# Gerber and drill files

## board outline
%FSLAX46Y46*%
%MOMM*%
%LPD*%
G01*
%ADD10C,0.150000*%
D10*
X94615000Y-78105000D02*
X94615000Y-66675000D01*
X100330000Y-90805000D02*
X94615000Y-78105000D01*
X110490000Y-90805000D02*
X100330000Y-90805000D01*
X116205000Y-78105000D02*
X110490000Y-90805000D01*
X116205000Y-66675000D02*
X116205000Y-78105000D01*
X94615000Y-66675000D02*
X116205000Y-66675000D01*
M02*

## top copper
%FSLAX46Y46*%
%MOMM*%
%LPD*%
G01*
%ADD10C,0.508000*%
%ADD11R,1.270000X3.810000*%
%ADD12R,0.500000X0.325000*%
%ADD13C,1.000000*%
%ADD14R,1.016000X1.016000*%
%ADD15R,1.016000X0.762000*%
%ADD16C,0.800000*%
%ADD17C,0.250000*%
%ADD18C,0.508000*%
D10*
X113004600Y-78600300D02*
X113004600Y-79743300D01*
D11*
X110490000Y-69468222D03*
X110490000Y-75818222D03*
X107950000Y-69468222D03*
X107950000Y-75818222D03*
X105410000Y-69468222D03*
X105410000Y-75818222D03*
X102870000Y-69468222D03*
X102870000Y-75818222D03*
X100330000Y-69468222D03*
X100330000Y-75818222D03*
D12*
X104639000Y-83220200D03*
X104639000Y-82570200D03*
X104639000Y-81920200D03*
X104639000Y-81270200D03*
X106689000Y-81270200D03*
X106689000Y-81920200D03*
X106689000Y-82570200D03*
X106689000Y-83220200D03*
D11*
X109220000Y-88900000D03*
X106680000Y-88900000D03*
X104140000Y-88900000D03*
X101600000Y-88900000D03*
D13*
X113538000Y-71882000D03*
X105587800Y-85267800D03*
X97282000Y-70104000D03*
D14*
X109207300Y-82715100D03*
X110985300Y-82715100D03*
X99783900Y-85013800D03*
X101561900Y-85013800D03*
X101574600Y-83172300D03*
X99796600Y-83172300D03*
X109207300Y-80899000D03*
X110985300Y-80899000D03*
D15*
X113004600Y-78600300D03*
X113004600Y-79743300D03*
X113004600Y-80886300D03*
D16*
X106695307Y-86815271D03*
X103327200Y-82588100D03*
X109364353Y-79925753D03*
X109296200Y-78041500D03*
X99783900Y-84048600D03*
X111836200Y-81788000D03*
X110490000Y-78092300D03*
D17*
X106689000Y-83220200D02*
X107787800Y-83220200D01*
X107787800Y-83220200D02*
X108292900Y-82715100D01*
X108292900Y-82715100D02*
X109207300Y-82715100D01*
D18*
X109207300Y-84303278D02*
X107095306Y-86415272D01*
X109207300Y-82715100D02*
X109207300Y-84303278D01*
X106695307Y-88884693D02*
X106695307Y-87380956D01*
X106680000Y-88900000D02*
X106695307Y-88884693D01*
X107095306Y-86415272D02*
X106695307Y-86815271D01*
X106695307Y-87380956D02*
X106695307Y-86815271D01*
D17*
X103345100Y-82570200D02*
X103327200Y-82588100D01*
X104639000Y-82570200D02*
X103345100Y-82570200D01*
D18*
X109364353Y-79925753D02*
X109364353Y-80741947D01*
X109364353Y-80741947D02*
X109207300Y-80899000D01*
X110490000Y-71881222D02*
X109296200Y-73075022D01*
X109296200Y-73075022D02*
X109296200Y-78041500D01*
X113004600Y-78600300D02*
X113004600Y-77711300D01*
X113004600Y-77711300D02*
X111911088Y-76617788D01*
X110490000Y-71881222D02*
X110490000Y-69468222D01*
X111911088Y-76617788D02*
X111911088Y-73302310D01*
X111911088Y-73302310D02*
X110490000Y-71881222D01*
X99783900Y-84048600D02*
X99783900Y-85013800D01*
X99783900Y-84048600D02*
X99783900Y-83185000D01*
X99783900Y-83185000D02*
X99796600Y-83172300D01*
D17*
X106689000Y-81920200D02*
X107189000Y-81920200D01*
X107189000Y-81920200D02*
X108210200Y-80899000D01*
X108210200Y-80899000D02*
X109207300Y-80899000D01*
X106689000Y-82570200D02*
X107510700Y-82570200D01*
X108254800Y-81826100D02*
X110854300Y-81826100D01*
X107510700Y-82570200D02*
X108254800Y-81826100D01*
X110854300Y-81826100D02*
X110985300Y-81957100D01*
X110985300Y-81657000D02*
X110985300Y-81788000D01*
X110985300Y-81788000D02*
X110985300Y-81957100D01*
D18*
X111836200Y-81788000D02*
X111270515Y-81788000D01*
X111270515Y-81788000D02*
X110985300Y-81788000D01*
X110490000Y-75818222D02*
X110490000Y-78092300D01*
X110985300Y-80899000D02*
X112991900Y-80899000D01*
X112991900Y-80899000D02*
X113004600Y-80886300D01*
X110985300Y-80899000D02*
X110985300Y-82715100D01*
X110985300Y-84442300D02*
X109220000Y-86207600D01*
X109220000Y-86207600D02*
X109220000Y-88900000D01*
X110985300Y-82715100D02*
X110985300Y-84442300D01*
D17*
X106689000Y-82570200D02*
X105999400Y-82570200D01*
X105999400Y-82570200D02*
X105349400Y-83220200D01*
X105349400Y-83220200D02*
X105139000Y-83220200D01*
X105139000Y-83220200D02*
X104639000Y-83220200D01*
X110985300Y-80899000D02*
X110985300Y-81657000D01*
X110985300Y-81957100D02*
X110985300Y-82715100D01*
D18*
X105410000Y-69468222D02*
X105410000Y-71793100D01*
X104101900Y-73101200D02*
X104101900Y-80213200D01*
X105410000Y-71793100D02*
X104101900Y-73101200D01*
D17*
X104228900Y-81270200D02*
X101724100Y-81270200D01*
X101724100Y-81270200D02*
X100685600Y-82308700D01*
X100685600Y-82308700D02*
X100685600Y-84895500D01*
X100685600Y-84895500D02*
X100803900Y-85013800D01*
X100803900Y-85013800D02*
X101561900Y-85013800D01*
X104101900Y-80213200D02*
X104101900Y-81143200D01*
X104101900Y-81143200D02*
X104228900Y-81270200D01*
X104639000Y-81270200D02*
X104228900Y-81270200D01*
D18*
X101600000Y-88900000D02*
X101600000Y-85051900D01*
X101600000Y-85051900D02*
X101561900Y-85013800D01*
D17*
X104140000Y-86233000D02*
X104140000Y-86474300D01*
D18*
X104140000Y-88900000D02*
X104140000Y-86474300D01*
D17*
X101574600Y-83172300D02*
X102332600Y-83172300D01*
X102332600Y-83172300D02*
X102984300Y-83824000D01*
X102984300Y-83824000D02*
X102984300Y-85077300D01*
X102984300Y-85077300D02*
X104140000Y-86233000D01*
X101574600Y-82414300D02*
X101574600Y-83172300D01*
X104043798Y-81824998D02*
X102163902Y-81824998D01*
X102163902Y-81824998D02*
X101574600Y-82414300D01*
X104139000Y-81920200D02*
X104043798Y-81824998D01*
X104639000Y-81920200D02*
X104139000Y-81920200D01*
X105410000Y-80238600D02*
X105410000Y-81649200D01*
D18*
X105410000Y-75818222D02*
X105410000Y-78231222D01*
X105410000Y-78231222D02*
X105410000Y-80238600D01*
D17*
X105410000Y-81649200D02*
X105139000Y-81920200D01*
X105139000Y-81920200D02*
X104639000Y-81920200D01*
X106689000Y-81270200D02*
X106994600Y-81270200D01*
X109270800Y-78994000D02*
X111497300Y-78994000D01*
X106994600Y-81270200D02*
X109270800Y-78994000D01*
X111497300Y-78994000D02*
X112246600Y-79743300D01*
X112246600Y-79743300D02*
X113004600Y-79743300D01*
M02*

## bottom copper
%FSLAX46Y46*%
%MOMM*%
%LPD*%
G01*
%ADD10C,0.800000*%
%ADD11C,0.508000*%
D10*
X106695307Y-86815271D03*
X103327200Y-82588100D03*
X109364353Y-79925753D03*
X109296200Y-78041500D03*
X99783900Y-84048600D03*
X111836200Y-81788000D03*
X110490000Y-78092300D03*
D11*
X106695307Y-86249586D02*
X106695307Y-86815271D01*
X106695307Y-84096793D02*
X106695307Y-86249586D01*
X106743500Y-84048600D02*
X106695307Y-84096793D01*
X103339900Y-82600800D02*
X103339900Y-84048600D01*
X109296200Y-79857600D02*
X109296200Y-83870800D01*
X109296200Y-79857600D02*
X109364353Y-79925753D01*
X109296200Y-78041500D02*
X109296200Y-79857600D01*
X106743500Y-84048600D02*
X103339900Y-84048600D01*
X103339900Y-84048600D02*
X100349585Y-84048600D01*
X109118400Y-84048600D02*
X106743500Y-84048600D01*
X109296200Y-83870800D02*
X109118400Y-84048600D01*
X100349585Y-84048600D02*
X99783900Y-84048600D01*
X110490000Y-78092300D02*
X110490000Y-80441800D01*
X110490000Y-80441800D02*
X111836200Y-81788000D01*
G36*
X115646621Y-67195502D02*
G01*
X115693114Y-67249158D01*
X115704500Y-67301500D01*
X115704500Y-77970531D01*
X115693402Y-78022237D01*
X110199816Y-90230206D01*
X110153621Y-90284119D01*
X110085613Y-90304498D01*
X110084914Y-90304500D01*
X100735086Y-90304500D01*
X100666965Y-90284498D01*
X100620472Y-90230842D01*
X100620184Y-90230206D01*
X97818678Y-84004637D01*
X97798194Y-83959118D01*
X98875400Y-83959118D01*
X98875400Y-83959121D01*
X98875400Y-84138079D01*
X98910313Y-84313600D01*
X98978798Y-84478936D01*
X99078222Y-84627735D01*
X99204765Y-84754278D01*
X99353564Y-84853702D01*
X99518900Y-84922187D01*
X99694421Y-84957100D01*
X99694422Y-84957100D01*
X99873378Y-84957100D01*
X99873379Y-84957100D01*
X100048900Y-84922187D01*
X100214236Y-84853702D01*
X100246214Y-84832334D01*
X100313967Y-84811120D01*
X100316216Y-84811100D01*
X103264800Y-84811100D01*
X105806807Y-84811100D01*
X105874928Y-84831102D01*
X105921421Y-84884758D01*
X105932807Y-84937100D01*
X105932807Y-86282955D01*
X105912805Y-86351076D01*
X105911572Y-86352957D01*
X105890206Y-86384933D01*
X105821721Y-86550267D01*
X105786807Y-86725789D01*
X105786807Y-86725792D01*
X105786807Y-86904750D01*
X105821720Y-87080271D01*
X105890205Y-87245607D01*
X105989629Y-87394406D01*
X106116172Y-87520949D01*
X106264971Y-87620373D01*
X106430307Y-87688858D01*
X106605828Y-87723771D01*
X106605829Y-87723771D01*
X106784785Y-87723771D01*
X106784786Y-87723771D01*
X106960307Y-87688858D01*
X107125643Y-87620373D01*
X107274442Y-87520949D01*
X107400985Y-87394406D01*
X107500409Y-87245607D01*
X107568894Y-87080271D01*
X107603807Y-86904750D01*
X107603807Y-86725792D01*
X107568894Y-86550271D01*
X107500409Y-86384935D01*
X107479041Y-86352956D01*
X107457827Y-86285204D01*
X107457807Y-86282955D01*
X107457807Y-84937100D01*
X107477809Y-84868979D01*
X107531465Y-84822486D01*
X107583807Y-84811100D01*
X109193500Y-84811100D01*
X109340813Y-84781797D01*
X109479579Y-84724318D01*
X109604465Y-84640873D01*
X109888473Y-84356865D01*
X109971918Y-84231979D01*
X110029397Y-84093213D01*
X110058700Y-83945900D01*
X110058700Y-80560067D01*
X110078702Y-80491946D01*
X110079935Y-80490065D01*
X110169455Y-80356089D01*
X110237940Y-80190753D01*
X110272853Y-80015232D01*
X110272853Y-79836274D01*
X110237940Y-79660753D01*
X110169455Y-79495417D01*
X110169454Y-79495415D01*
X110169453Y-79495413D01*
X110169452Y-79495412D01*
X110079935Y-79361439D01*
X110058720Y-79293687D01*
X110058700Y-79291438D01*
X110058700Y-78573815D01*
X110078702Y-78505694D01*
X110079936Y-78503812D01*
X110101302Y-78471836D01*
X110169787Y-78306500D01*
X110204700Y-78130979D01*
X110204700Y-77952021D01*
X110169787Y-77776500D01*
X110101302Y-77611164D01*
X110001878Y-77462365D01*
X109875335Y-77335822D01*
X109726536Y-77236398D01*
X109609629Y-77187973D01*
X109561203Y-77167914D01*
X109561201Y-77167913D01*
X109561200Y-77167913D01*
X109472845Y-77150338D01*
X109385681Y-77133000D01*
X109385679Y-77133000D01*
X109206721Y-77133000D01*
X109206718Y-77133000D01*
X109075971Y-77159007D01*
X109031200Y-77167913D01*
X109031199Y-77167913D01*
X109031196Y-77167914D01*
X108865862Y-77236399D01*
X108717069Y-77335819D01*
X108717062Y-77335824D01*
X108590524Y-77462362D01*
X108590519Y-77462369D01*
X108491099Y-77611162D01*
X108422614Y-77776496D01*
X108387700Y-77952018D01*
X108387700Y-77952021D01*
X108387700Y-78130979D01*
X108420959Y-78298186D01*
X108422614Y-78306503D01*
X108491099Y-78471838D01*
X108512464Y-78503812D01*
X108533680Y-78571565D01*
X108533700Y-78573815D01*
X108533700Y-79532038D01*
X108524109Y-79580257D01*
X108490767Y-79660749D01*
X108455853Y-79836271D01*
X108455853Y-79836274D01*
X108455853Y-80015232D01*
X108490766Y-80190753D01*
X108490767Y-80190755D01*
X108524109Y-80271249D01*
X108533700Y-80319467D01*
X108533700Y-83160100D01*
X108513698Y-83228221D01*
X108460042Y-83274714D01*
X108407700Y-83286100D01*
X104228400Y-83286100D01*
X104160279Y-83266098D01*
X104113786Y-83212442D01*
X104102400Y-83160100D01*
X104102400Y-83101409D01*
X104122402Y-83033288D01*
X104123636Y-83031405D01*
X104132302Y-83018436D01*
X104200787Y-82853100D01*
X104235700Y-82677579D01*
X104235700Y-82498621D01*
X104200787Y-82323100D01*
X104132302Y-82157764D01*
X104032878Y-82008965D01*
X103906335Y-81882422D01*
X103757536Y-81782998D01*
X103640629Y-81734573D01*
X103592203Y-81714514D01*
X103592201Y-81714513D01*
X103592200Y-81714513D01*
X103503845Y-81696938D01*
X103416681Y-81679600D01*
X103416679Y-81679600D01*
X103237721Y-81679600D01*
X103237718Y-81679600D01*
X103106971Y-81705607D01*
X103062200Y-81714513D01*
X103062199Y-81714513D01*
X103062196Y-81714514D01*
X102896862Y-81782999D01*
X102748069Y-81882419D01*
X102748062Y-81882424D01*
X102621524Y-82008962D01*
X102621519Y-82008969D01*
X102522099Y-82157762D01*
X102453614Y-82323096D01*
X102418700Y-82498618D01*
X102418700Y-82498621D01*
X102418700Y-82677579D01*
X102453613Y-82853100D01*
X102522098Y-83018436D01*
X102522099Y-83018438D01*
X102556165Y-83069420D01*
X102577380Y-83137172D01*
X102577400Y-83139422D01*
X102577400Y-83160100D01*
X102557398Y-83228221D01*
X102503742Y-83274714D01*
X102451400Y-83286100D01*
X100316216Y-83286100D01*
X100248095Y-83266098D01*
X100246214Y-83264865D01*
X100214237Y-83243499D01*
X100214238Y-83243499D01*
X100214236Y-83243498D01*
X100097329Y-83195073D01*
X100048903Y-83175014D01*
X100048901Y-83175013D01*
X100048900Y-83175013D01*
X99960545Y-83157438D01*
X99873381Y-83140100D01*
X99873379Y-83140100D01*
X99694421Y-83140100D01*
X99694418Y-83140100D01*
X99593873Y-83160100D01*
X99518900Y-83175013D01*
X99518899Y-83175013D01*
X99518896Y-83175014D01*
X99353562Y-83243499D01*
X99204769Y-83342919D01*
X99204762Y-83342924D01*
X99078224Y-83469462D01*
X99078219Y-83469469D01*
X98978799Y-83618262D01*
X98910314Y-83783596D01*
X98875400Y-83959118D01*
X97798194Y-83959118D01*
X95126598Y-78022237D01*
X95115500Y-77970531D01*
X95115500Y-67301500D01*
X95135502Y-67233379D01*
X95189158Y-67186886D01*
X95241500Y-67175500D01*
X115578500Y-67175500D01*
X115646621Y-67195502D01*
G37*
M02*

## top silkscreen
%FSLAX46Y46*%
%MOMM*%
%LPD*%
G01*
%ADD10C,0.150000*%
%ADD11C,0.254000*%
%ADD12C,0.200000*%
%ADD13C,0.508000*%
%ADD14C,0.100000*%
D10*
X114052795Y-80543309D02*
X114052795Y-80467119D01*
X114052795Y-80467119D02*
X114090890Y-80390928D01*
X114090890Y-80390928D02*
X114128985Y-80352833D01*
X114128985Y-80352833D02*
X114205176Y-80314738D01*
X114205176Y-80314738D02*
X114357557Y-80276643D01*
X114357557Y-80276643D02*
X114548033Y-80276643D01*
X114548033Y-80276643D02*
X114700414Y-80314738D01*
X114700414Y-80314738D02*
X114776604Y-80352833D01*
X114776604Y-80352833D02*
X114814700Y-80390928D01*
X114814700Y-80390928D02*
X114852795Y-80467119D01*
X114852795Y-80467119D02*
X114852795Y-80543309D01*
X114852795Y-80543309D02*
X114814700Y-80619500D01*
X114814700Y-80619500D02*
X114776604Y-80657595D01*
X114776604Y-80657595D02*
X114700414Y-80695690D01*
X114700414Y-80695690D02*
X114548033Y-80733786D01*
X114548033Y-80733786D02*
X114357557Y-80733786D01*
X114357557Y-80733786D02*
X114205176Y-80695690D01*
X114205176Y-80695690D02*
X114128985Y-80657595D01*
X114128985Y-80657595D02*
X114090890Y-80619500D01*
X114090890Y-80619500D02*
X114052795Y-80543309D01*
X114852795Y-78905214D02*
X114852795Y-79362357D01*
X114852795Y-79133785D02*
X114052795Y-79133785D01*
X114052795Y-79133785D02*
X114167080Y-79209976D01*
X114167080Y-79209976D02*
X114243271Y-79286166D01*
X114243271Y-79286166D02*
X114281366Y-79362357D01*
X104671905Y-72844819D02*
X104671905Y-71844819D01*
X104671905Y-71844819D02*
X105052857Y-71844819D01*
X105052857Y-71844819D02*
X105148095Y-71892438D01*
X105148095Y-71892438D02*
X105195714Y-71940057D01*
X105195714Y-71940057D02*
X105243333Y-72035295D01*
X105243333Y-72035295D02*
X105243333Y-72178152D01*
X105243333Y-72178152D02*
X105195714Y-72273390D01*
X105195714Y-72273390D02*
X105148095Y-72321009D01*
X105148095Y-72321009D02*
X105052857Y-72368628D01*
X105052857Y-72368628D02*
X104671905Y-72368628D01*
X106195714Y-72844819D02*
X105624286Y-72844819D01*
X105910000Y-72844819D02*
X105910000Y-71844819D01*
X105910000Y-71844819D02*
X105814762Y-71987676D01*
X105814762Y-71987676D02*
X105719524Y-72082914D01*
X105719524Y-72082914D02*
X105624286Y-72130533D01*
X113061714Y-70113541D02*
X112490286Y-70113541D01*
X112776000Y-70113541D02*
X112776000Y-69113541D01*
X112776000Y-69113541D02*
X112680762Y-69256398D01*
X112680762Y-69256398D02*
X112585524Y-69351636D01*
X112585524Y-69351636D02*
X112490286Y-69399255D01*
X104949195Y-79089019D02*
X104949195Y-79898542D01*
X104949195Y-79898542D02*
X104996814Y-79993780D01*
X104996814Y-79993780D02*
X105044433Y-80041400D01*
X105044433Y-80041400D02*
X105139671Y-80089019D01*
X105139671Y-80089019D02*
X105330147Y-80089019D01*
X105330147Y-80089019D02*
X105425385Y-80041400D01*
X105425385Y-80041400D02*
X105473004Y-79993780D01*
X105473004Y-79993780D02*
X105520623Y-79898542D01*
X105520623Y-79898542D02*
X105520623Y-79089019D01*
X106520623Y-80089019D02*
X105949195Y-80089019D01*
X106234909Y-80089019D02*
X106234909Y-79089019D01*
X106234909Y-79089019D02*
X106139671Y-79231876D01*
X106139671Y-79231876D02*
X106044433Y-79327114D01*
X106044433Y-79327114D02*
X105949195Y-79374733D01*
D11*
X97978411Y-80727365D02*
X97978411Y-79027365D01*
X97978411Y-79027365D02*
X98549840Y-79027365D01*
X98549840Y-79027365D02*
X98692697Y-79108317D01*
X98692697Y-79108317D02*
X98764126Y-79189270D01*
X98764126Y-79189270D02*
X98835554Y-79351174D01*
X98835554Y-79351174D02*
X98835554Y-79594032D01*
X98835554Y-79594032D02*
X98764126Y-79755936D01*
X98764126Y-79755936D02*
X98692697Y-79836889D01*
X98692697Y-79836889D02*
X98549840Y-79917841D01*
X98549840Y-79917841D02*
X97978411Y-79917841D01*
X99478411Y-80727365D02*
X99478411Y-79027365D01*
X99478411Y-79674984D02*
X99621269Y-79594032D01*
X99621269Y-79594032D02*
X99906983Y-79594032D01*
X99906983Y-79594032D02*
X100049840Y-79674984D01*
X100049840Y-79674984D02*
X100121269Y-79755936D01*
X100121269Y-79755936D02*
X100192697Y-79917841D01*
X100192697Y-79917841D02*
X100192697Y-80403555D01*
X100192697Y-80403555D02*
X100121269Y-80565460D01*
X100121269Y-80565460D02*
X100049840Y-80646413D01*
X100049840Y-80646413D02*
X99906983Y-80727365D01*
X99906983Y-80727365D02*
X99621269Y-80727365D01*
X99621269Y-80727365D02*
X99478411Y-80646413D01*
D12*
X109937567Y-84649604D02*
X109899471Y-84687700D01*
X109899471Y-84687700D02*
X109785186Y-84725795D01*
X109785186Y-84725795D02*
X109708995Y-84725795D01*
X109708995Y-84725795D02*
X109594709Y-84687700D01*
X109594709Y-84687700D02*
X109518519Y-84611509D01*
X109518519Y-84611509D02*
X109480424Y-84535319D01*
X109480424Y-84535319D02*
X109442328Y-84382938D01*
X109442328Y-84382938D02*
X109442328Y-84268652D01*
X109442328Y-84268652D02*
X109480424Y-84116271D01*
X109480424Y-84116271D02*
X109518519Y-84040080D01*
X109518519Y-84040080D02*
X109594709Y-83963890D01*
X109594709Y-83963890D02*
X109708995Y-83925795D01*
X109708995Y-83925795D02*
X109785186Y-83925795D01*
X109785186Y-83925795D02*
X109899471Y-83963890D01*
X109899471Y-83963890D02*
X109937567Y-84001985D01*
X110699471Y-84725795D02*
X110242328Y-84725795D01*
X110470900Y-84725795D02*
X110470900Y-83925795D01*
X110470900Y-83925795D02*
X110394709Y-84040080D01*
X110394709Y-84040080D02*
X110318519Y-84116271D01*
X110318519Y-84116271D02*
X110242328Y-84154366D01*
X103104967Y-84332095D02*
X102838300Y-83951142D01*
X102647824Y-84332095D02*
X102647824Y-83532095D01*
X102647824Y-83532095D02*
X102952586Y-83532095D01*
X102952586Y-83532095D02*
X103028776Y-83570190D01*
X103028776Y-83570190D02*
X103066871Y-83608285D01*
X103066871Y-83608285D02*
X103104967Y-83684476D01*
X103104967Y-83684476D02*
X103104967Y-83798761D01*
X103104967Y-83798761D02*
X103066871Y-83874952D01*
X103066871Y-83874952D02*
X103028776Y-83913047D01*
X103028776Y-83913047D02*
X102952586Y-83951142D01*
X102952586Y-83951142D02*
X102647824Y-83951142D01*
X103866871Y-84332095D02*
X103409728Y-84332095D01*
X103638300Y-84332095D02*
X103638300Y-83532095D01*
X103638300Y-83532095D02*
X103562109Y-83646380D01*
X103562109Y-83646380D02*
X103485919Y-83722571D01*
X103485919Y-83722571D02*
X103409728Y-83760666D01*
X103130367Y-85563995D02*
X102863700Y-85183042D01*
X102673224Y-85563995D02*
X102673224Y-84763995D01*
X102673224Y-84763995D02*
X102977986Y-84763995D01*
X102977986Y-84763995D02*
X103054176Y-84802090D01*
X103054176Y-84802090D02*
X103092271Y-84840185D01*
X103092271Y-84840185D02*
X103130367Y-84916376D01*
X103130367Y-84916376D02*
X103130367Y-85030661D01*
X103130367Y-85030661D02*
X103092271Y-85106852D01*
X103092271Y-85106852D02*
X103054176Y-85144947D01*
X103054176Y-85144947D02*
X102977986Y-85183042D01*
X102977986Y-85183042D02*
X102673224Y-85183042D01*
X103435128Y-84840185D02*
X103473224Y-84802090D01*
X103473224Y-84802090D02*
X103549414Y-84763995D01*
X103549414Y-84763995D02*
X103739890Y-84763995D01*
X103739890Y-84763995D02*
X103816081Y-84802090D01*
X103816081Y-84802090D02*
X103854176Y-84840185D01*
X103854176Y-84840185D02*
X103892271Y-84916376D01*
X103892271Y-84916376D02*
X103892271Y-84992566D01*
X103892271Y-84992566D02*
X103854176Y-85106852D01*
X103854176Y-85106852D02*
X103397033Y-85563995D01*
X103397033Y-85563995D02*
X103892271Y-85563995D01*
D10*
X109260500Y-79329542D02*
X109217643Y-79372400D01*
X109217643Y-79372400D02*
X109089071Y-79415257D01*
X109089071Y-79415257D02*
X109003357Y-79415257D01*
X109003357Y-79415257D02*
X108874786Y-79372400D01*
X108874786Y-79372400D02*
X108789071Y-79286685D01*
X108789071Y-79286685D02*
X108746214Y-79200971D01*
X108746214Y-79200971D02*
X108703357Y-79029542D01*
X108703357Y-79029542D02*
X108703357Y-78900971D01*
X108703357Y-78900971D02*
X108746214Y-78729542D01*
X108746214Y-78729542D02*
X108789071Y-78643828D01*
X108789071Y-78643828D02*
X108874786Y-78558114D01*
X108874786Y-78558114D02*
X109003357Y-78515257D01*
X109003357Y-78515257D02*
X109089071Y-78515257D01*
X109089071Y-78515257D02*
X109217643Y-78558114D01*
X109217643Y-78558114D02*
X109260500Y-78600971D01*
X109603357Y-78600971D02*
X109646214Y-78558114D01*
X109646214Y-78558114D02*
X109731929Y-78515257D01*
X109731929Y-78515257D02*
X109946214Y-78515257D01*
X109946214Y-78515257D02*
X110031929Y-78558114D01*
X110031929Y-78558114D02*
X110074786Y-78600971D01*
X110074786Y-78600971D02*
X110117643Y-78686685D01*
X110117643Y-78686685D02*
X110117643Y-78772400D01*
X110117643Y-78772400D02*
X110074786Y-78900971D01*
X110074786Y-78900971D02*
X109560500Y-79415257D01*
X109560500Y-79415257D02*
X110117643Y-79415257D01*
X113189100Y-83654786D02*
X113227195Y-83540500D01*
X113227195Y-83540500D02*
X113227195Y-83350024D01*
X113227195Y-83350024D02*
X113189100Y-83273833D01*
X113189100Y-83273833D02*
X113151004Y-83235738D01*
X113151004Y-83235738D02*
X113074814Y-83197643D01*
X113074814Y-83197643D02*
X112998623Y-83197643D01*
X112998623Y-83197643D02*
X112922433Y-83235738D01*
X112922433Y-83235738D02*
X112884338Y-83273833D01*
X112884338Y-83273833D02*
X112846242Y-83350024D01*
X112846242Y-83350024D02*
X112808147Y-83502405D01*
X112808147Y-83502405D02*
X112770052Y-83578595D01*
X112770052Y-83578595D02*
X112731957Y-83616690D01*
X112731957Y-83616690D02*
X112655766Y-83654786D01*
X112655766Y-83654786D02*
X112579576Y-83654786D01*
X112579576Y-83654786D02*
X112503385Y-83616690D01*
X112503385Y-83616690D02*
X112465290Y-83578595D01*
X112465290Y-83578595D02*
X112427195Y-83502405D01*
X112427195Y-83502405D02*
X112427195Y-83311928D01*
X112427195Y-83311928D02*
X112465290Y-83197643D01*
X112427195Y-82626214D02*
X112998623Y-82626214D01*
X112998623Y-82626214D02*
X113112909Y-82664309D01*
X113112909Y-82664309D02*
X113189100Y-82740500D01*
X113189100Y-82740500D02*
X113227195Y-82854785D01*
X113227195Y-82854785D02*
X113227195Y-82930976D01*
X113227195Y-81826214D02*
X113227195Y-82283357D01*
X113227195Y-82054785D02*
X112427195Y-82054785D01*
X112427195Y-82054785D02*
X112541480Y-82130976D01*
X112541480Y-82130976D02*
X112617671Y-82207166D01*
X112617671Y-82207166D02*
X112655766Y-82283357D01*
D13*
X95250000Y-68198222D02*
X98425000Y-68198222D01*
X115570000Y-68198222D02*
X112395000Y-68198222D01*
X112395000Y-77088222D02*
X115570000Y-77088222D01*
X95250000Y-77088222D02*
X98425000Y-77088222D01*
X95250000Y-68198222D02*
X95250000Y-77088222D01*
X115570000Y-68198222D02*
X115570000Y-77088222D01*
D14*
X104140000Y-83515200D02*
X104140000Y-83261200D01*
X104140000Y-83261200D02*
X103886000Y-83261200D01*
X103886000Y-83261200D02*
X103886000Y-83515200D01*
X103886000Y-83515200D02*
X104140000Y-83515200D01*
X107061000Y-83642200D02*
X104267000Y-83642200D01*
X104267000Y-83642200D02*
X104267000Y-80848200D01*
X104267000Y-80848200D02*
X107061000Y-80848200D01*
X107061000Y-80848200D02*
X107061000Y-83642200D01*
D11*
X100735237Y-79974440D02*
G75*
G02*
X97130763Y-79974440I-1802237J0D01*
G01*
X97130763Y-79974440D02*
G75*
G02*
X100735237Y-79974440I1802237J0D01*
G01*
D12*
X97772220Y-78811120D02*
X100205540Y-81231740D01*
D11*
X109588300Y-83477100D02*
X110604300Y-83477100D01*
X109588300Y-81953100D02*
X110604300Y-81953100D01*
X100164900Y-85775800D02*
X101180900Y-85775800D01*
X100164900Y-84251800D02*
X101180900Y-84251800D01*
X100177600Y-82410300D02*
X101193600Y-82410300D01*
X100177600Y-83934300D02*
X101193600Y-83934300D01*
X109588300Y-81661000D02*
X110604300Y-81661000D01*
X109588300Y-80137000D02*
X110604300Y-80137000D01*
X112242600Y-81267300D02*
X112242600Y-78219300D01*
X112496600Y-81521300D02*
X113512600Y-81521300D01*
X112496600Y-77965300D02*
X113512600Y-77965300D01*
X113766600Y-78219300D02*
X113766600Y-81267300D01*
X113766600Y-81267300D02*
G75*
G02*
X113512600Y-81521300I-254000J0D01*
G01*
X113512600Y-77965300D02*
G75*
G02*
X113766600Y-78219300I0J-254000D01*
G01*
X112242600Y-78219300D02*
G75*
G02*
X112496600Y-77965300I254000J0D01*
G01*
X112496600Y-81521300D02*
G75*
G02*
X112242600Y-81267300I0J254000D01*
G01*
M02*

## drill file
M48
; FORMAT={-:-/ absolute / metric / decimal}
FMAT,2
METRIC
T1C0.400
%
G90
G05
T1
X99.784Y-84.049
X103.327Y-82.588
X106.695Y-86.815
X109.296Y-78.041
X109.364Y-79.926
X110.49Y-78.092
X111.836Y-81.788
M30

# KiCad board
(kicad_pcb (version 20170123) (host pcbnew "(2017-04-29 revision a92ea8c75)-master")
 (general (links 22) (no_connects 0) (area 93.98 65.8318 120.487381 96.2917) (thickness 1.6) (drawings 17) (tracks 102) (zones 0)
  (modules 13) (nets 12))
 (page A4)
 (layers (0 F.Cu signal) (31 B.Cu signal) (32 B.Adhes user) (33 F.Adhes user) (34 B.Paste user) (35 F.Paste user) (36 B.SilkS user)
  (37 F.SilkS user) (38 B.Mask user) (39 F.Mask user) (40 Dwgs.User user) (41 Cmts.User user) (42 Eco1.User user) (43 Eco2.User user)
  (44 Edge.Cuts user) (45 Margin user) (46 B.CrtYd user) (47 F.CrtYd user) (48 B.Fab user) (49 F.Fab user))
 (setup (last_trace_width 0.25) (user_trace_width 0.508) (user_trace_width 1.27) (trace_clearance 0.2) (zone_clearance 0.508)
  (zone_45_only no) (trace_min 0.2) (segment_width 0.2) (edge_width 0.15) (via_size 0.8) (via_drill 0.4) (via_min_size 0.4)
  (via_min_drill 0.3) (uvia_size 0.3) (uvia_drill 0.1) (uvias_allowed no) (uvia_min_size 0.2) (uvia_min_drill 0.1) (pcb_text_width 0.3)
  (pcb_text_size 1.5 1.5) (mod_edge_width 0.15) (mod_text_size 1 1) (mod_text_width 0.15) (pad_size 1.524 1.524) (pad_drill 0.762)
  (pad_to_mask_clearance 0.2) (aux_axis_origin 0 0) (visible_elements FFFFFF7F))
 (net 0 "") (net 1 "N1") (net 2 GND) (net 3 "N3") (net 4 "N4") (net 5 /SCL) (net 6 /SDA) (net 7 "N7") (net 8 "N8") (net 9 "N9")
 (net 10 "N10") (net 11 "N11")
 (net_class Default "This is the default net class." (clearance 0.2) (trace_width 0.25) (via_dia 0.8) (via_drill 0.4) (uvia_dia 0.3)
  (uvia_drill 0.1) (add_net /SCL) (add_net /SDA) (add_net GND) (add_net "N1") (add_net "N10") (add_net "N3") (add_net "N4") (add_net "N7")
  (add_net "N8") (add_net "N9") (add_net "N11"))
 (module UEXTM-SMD (layer F.Cu) (at 105.41 72.643222)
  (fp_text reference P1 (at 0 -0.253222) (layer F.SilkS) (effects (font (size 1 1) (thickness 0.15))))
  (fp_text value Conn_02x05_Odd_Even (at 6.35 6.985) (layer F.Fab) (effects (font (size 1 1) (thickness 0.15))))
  (fp_line (start -10.16 -4.445) (end -6.985 -4.445) (layer F.SilkS) (width 0.508))
  (fp_line (start 10.16 -4.445) (end 6.985 -4.445) (layer F.SilkS) (width 0.508))
  (fp_line (start 6.985 4.445) (end 10.16 4.445) (layer F.SilkS) (width 0.508))
  (fp_line (start -10.16 4.445) (end -6.985 4.445) (layer F.SilkS) (width 0.508))
  (fp_line (start -10.16 -4.445) (end -10.16 4.445) (layer F.SilkS) (width 0.508))
  (fp_line (start 10.16 -4.445) (end 10.16 4.445) (layer F.SilkS) (width 0.508))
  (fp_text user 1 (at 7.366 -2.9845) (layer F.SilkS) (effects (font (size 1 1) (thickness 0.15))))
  (pad 1 smd rect (at 5.08 -3.175) (size 1.27 3.81) (layers F.Cu F.Paste F.Mask) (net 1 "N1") (solder_mask_margin 0.0508)
   (solder_paste_margin 0.0508) (clearance 0.0508))
  (pad 2 smd rect (at 5.08 3.175) (size 1.27 3.81) (layers F.Cu F.Paste F.Mask) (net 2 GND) (solder_mask_margin 0.0508)
   (solder_paste_margin 0.0508) (clearance 0.0508))
  (pad 3 smd rect (at 2.54 -3.175) (size 1.27 3.81) (layers F.Cu F.Paste F.Mask) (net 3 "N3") (solder_mask_margin 0.0508)
   (solder_paste_margin 0.0508) (clearance 0.0508))
  (pad 4 smd rect (at 2.54 3.175) (size 1.27 3.81) (layers F.Cu F.Paste F.Mask) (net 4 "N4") (solder_mask_margin 0.0508)
   (solder_paste_margin 0.0508) (clearance 0.0508))
  (pad 5 smd rect (at 0 -3.175) (size 1.27 3.81) (layers F.Cu F.Paste F.Mask) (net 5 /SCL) (solder_mask_margin 0.0508)
   (solder_paste_margin 0.0508) (clearance 0.0508))
  (pad 6 smd rect (at 0 3.175) (size 1.27 3.81) (layers F.Cu F.Paste F.Mask) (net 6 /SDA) (solder_mask_margin 0.0508)
   (solder_paste_margin 0.0508) (clearance 0.0508))
  (pad 7 smd rect (at -2.54 -3.175) (size 1.27 3.81) (layers F.Cu F.Paste F.Mask) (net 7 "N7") (solder_mask_margin 0.0508)
   (solder_paste_margin 0.0508) (clearance 0.0508))
  (pad 8 smd rect (at -2.54 3.175) (size 1.27 3.81) (layers F.Cu F.Paste F.Mask) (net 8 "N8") (solder_mask_margin 0.0508)
   (solder_paste_margin 0.0508) (clearance 0.0508))
  (pad 9 smd rect (at -5.08 -3.175) (size 1.27 3.81) (layers F.Cu F.Paste F.Mask) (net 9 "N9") (solder_mask_margin 0.0508)
   (solder_paste_margin 0.0508) (clearance 0.0508))
  (pad 10 smd rect (at -5.08 3.175) (size 1.27 3.81) (layers F.Cu F.Paste F.Mask) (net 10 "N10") (solder_mask_margin 0.0508)
   (solder_paste_margin 0.0508) (clearance 0.0508)))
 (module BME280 (layer F.Cu) (at 105.664 82.2452 180)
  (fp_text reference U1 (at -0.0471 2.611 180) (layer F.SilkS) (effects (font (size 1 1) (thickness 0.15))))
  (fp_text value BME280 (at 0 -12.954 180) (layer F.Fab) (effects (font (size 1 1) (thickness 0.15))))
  (fp_line (start 1.524 -1.27) (end 1.524 -1.016) (layer F.SilkS) (width 0.1))
  (fp_line (start 1.524 -1.016) (end 1.778 -1.016) (layer F.SilkS) (width 0.1))
  (fp_line (start 1.778 -1.016) (end 1.778 -1.27) (layer F.SilkS) (width 0.1))
  (fp_line (start 1.778 -1.27) (end 1.524 -1.27) (layer F.SilkS) (width 0.1))
  (fp_line (start -1.397 -1.397) (end 1.397 -1.397) (layer F.SilkS) (width 0.1))
  (fp_line (start 1.397 -1.397) (end 1.397 1.397) (layer F.SilkS) (width 0.1))
  (fp_line (start 1.397 1.397) (end -1.397 1.397) (layer F.SilkS) (width 0.1))
  (fp_line (start -1.397 1.397) (end -1.397 -1.397) (layer F.SilkS) (width 0.1))
  (pad 1 smd rect (at 1.025 -0.975 180) (size 0.5 0.325) (layers F.Cu F.Paste F.Mask) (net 2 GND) (solder_mask_margin 0.05))
  (pad 2 smd rect (at 1.025 -0.325 180) (size 0.5 0.325) (layers F.Cu F.Paste F.Mask) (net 1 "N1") (solder_mask_margin 0.05))
  (pad 3 smd rect (at 1.025 0.325 180) (size 0.5 0.325) (layers F.Cu F.Paste F.Mask) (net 6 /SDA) (solder_mask_margin 0.05))
  (pad 4 smd rect (at 1.025 0.975 180) (size 0.5 0.325) (layers F.Cu F.Paste F.Mask) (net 5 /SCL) (solder_mask_margin 0.05))
  (pad 5 smd rect (at -1.025 0.975 180) (size 0.5 0.325) (layers F.Cu F.Paste F.Mask) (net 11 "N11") (solder_mask_margin 0.05))
  (pad 6 smd rect (at -1.025 0.325 180) (size 0.5 0.325) (layers F.Cu F.Paste F.Mask) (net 1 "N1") (solder_mask_margin 0.05))
  (pad 7 smd rect (at -1.025 -0.325 180) (size 0.5 0.325) (layers F.Cu F.Paste F.Mask) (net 2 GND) (solder_mask_margin 0.05))
  (pad 8 smd rect (at -1.025 -0.975 180) (size 0.5 0.325) (layers F.Cu F.Paste F.Mask) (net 1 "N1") (solder_mask_margin 0.05)))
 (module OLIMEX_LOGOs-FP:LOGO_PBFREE (layer F.Cu) (at 99.1362 80.2894)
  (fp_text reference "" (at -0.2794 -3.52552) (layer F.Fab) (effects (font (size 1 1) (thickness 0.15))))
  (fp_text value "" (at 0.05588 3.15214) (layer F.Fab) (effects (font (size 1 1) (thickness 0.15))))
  (fp_circle (center -0.2032 -0.31496) (end 0.90678 -1.73482) (layer F.SilkS) (width 0.254))
  (fp_line (start -1.36398 -1.47828) (end 1.06934 0.94234) (layer F.SilkS) (width 0.2))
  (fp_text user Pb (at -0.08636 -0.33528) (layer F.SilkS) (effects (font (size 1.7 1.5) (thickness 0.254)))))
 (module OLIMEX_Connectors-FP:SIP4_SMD (layer F.Cu) (at 105.41 88.9 180)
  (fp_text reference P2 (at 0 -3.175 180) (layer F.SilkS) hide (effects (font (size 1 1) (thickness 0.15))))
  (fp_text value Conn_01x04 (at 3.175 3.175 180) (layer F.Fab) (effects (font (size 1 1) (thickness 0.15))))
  (pad 1 smd rect (at -3.81 0 180) (size 1.27 3.81) (layers F.Cu F.Mask) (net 2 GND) (solder_mask_margin 0.0508)
   (solder_paste_margin -0.0508) (clearance 0.0508))
  (pad 2 smd rect (at -1.27 0 180) (size 1.27 3.81) (layers F.Cu F.Mask) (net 1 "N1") (solder_mask_margin 0.0508)
   (solder_paste_margin -0.0508) (clearance 0.0508))
  (pad 3 smd rect (at 1.27 0 180) (size 1.27 3.81) (layers F.Cu F.Mask) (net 6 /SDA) (solder_mask_margin 0.0508)
   (solder_paste_margin -0.0508) (clearance 0.0508))
  (pad 4 smd rect (at 3.81 0 180) (size 1.27 3.81) (layers F.Cu F.Mask) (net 5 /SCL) (solder_mask_margin 0.0508)
   (solder_paste_margin -0.0508) (clearance 0.0508)))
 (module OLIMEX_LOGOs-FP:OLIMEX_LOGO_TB (layer B.Cu) (at 105.41 69.85 180)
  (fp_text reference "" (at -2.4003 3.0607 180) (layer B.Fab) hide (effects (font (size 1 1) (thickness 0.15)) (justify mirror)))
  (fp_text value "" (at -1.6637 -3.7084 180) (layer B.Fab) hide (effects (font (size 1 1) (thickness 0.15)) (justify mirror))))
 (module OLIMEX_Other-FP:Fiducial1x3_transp (layer F.Cu) (at 113.538 71.882)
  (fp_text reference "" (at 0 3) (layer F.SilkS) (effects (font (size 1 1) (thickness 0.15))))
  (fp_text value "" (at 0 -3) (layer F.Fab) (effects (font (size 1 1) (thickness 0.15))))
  (pad Fid1 connect circle (at 0 0) (size 1 1) (layers F.Cu F.Mask) (solder_mask_margin 0.127) (clearance 1.016) (zone_connect 0)))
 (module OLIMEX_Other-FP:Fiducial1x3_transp (layer F.Cu) (at 105.5878 85.2678)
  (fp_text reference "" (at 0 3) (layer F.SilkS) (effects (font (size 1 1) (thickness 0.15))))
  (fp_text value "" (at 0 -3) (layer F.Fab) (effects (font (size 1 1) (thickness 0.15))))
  (pad Fid1 connect circle (at 0 0) (size 1 1) (layers F.Cu F.Mask) (solder_mask_margin 0.127) (clearance 1.016) (zone_connect 0)))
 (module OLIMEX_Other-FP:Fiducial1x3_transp (layer F.Cu) (at 97.282 70.104)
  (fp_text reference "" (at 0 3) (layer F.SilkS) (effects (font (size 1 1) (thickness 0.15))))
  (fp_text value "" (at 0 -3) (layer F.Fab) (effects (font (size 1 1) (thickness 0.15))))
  (pad Fid1 connect circle (at 0 0) (size 1 1) (layers F.Cu F.Mask) (solder_mask_margin 0.127) (clearance 1.016) (zone_connect 0)))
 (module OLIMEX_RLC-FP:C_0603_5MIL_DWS (layer F.Cu) (at 110.0963 82.7151)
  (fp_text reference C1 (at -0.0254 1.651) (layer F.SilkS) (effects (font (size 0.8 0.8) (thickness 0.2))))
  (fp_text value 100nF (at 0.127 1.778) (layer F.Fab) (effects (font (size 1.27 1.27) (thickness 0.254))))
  (fp_line (start -0.508 0.762) (end 0.508 0.762) (layer F.SilkS) (width 0.254))
  (fp_line (start -0.508 -0.762) (end 0.508 -0.762) (layer F.SilkS) (width 0.254))
  (pad 1 smd rect (at -0.889 0) (size 1.016 1.016) (layers F.Cu F.Paste F.Mask) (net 1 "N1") (solder_mask_margin 0.0508) (clearance 0.0508))
  (pad 2 smd rect (at 0.889 0) (size 1.016 1.016) (layers F.Cu F.Paste F.Mask) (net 2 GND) (solder_mask_margin 0.0508) (clearance 0.0508)))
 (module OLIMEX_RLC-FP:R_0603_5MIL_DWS (layer F.Cu) (at 100.6729 85.0138)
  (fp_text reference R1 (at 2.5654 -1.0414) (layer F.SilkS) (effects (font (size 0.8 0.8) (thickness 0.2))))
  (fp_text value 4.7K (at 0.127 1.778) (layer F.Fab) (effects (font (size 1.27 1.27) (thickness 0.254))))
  (fp_line (start -0.508 0.762) (end 0.508 0.762) (layer F.SilkS) (width 0.254))
  (fp_line (start -0.508 -0.762) (end 0.508 -0.762) (layer F.SilkS) (width 0.254))
  (pad 1 smd rect (at -0.889 0) (size 1.016 1.016) (layers F.Cu F.Paste F.Mask) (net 1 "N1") (solder_mask_margin 0.0508))
  (pad 2 smd rect (at 0.889 0) (size 1.016 1.016) (layers F.Cu F.Paste F.Mask) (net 5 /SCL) (solder_mask_margin 0.0508)))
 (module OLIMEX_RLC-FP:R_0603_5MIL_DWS (layer F.Cu) (at 100.6856 83.1723)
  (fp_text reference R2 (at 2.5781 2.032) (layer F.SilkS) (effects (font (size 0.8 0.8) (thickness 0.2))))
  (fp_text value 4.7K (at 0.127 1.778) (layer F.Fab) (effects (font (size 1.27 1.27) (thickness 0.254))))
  (fp_line (start -0.508 -0.762) (end 0.508 -0.762) (layer F.SilkS) (width 0.254))
  (fp_line (start -0.508 0.762) (end 0.508 0.762) (layer F.SilkS) (width 0.254))
  (pad 2 smd rect (at 0.889 0) (size 1.016 1.016) (layers F.Cu F.Paste F.Mask) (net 6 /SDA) (solder_mask_margin 0.0508))
  (pad 1 smd rect (at -0.889 0) (size 1.016 1.016) (layers F.Cu F.Paste F.Mask) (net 1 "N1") (solder_mask_margin 0.0508)))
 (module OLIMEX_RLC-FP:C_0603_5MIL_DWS (layer F.Cu) (at 110.0963 80.899)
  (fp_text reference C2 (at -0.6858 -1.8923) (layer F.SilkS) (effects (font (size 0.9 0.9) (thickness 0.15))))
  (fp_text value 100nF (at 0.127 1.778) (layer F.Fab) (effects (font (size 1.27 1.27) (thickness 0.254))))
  (fp_line (start -0.508 0.762) (end 0.508 0.762) (layer F.SilkS) (width 0.254))
  (fp_line (start -0.508 -0.762) (end 0.508 -0.762) (layer F.SilkS) (width 0.254))
  (pad 1 smd rect (at -0.889 0) (size 1.016 1.016) (layers F.Cu F.Paste F.Mask) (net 1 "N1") (solder_mask_margin 0.0508) (clearance 0.0508))
  (pad 2 smd rect (at 0.889 0) (size 1.016 1.016) (layers F.Cu F.Paste F.Mask) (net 2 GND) (solder_mask_margin 0.0508) (clearance 0.0508)))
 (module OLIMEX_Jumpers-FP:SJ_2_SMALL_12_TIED (layer F.Cu) (at 113.0046 79.7433 270)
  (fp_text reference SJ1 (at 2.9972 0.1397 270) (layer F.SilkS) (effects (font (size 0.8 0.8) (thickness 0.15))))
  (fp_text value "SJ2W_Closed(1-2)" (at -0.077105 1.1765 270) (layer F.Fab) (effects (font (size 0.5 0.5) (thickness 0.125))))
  (fp_line (start 1.524 0.762) (end -1.524 0.762) (layer F.SilkS) (width 0.254))
  (fp_line (start 1.778 0.508) (end 1.778 -0.508) (layer F.SilkS) (width 0.254))
  (fp_line (start -1.778 0.508) (end -1.778 -0.508) (layer F.SilkS) (width 0.254))
  (fp_line (start -1.524 -0.762) (end 1.524 -0.762) (layer F.SilkS) (width 0.254))
  (fp_line (start -1.143 0) (end 0 0) (layer F.Cu) (width 0.508))
  (fp_arc (start 1.524 -0.508) (end 1.524 -0.762) (angle 90) (layer F.SilkS) (width 0.254))
  (fp_arc (start -1.524 -0.508) (end -1.778 -0.508) (angle 90) (layer F.SilkS) (width 0.254))
  (fp_arc (start -1.524 0.508) (end -1.524 0.762) (angle 90) (layer F.SilkS) (width 0.254))
  (fp_arc (start 1.524 0.508) (end 1.778 0.508) (angle 90) (layer F.SilkS) (width 0.254))
  (pad 1 smd rect (at -1.143 0 270) (size 0.762 1.016) (layers F.Cu F.Mask) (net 1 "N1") (solder_mask_margin 0.0508)
   (solder_paste_margin -0.0508) (clearance 0.0508))
  (pad 2 smd rect (at 0 0 270) (size 0.762 1.016) (layers F.Cu F.Mask) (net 11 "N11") (solder_mask_margin 0.0508)
   (solder_paste_margin -0.0508) (clearance 0.0508))
  (pad 3 smd rect (at 1.143 0 270) (size 0.762 1.016) (layers F.Cu F.Mask) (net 2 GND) (solder_mask_margin 0.0508)
   (solder_paste_margin -0.0508) (clearance 0.0508)))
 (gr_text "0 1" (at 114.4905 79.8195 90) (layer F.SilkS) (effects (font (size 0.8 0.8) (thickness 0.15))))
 (gr_line (start 94.615 78.105) (end 94.615 66.675) (layer Edge.Cuts) (width 0.15))
 (gr_line (start 100.33 90.805) (end 94.615 78.105) (layer Edge.Cuts) (width 0.15))
 (gr_line (start 110.49 90.805) (end 100.33 90.805) (layer Edge.Cuts) (width 0.15))
 (gr_line (start 116.205 78.105) (end 110.49 90.805) (layer Edge.Cuts) (width 0.15))
 (gr_line (start 116.205 66.675) (end 116.205 78.105) (layer Edge.Cuts) (width 0.15))
 (gr_line (start 94.615 66.675) (end 116.205 66.675) (layer Edge.Cuts) (width 0.15))
 (segment (start 106.689 83.2202) (end 107.7878 83.2202) (width 0.25) (layer F.Cu) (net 1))
 (segment (start 107.7878 83.2202) (end 108.2929 82.7151) (width 0.25) (layer F.Cu) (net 1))
 (segment (start 108.2929 82.7151) (end 109.2073 82.7151) (width 0.25) (layer F.Cu) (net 1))
 (segment (start 109.2073 84.303278) (end 107.095306 86.415272) (width 0.508) (layer F.Cu) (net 1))
 (segment (start 109.2073 82.7151) (end 109.2073 84.303278) (width 0.508) (layer F.Cu) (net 1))
 (segment (start 106.695307 88.884693) (end 106.695307 87.380956) (width 0.508) (layer F.Cu) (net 1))
 (segment (start 106.68 88.9) (end 106.695307 88.884693) (width 0.508) (layer F.Cu) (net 1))
 (segment (start 106.695307 86.249586) (end 106.695307 86.815271) (width 0.508) (layer B.Cu) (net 1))
 (segment (start 106.695307 84.096793) (end 106.695307 86.249586) (width 0.508) (layer B.Cu) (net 1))
 (segment (start 106.7435 84.0486) (end 106.695307 84.096793) (width 0.508) (layer B.Cu) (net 1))
 (segment (start 107.095306 86.415272) (end 106.695307 86.815271) (width 0.508) (layer F.Cu) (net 1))
 (segment (start 106.695307 87.380956) (end 106.695307 86.815271) (width 0.508) (layer F.Cu) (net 1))
 (via (at 106.695307 86.815271) (size 0.8) (drill 0.4) (layers F.Cu B.Cu) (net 1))
 (segment (start 103.3451 82.5702) (end 103.3272 82.5881) (width 0.25) (layer F.Cu) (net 1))
 (segment (start 104.639 82.5702) (end 103.3451 82.5702) (width 0.25) (layer F.Cu) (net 1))
 (via (at 103.3272 82.5881) (size 0.8) (drill 0.4) (layers F.Cu B.Cu) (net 1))
 (segment (start 103.3399 82.6008) (end 103.3399 84.0486) (width 0.508) (layer B.Cu) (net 1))
 (segment (start 109.364353 79.925753) (end 109.364353 80.741947) (width 0.508) (layer F.Cu) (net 1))
 (segment (start 109.364353 80.741947) (end 109.2073 80.899) (width 0.508) (layer F.Cu) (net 1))
 (segment (start 109.2962 79.8576) (end 109.2962 83.8708) (width 0.508) (layer B.Cu) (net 1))
 (segment (start 109.2962 79.8576) (end 109.364353 79.925753) (width 0.508) (layer B.Cu) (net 1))
 (segment (start 109.2962 78.0415) (end 109.2962 79.8576) (width 0.508) (layer B.Cu) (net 1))
 (via (at 109.364353 79.925753) (size 0.8) (drill 0.4) (layers F.Cu B.Cu) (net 1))
 (segment (start 106.7435 84.0486) (end 103.3399 84.0486) (width 0.508) (layer B.Cu) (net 1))
 (segment (start 103.3399 84.0486) (end 100.349585 84.0486) (width 0.508) (layer B.Cu) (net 1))
 (segment (start 109.1184 84.0486) (end 106.7435 84.0486) (width 0.508) (layer B.Cu) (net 1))
 (segment (start 109.2962 83.8708) (end 109.1184 84.0486) (width 0.508) (layer B.Cu) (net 1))
 (segment (start 100.349585 84.0486) (end 99.7839 84.0486) (width 0.508) (layer B.Cu) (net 1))
 (segment (start 110.49 71.881222) (end 109.2962 73.075022) (width 0.508) (layer F.Cu) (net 1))
 (segment (start 109.2962 73.075022) (end 109.2962 78.0415) (width 0.508) (layer F.Cu) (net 1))
 (via (at 109.2962 78.0415) (size 0.8) (drill 0.4) (layers F.Cu B.Cu) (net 1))
 (segment (start 113.0046 78.6003) (end 113.0046 77.7113) (width 0.508) (layer F.Cu) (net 1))
 (segment (start 113.0046 77.7113) (end 111.911088 76.617788) (width 0.508) (layer F.Cu) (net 1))
 (segment (start 110.49 71.881222) (end 110.49 69.468222) (width 0.508) (layer F.Cu) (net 1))
 (segment (start 111.911088 76.617788) (end 111.911088 73.30231) (width 0.508) (layer F.Cu) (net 1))
 (segment (start 111.911088 73.30231) (end 110.49 71.881222) (width 0.508) (layer F.Cu) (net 1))
 (segment (start 99.7839 84.0486) (end 99.7839 85.0138) (width 0.508) (layer F.Cu) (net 1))
 (segment (start 99.7839 84.0486) (end 99.7839 83.185) (width 0.508) (layer F.Cu) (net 1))
 (segment (start 99.7839 83.185) (end 99.7966 83.1723) (width 0.508) (layer F.Cu) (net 1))
 (via (at 99.7839 84.0486) (size 0.8) (drill 0.4) (layers F.Cu B.Cu) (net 1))
 (segment (start 106.689 81.9202) (end 107.189 81.9202) (width 0.25) (layer F.Cu) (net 1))
 (segment (start 107.189 81.9202) (end 108.2102 80.899) (width 0.25) (layer F.Cu) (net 1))
 (segment (start 108.2102 80.899) (end 109.2073 80.899) (width 0.25) (layer F.Cu) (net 1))
 (segment (start 106.689 82.5702) (end 107.5107 82.5702) (width 0.25) (layer F.Cu) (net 2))
 (segment (start 108.2548 81.8261) (end 110.8543 81.8261) (width 0.25) (layer F.Cu) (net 2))
 (segment (start 107.5107 82.5702) (end 108.2548 81.8261) (width 0.25) (layer F.Cu) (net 2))
 (segment (start 110.8543 81.8261) (end 110.9853 81.9571) (width 0.25) (layer F.Cu) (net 2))
 (segment (start 110.9853 81.657) (end 110.9853 81.788) (width 0.25) (layer F.Cu) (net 2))
 (segment (start 110.9853 81.788) (end 110.9853 81.9571) (width 0.25) (layer F.Cu) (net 2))
 (segment (start 111.8362 81.788) (end 111.270515 81.788) (width 0.508) (layer F.Cu) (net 2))
 (segment (start 111.270515 81.788) (end 110.9853 81.788) (width 0.508) (layer F.Cu) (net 2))
 (segment (start 110.49 78.0923) (end 110.49 80.4418) (width 0.508) (layer B.Cu) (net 2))
 (segment (start 110.49 80.4418) (end 111.8362 81.788) (width 0.508) (layer B.Cu) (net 2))
 (via (at 111.8362 81.788) (size 0.8) (drill 0.4) (layers F.Cu B.Cu) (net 2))
 (segment (start 110.49 75.818222) (end 110.49 78.0923) (width 0.508) (layer F.Cu) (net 2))
 (via (at 110.49 78.0923) (size 0.8) (drill 0.4) (layers F.Cu B.Cu) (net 2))
 (segment (start 110.9853 80.899) (end 112.9919 80.899) (width 0.508) (layer F.Cu) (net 2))
 (segment (start 112.9919 80.899) (end 113.0046 80.8863) (width 0.508) (layer F.Cu) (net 2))
 (segment (start 110.9853 80.899) (end 110.9853 82.7151) (width 0.508) (layer F.Cu) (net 2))
 (segment (start 110.9853 84.4423) (end 109.22 86.2076) (width 0.508) (layer F.Cu) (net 2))
 (segment (start 109.22 86.2076) (end 109.22 88.9) (width 0.508) (layer F.Cu) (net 2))
 (segment (start 110.9853 82.7151) (end 110.9853 84.4423) (width 0.508) (layer F.Cu) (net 2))
 (segment (start 106.689 82.5702) (end 105.9994 82.5702) (width 0.25) (layer F.Cu) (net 2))
 (segment (start 105.9994 82.5702) (end 105.3494 83.2202) (width 0.25) (layer F.Cu) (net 2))
 (segment (start 105.3494 83.2202) (end 105.139 83.2202) (width 0.25) (layer F.Cu) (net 2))
 (segment (start 105.139 83.2202) (end 104.639 83.2202) (width 0.25) (layer F.Cu) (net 2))
 (segment (start 110.9853 80.899) (end 110.9853 81.657) (width 0.25) (layer F.Cu) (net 2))
 (segment (start 110.9853 81.9571) (end 110.9853 82.7151) (width 0.25) (layer F.Cu) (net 2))
 (segment (start 105.41 69.468222) (end 105.41 71.7931) (width 0.508) (layer F.Cu) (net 5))
 (segment (start 104.1019 73.1012) (end 104.1019 80.2132) (width 0.508) (layer F.Cu) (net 5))
 (segment (start 105.41 71.7931) (end 104.1019 73.1012) (width 0.508) (layer F.Cu) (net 5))
 (segment (start 104.2289 81.2702) (end 101.7241 81.2702) (width 0.25) (layer F.Cu) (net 5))
 (segment (start 101.7241 81.2702) (end 100.6856 82.3087) (width 0.25) (layer F.Cu) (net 5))
 (segment (start 100.6856 82.3087) (end 100.6856 84.8955) (width 0.25) (layer F.Cu) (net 5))
 (segment (start 100.6856 84.8955) (end 100.8039 85.0138) (width 0.25) (layer F.Cu) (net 5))
 (segment (start 100.8039 85.0138) (end 101.5619 85.0138) (width 0.25) (layer F.Cu) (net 5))
 (segment (start 104.1019 80.2132) (end 104.1019 81.1432) (width 0.25) (layer F.Cu) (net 5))
 (segment (start 104.1019 81.1432) (end 104.2289 81.2702) (width 0.25) (layer F.Cu) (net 5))
 (segment (start 104.639 81.2702) (end 104.2289 81.2702) (width 0.25) (layer F.Cu) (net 5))
 (segment (start 101.6 88.9) (end 101.6 85.0519) (width 0.508) (layer F.Cu) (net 5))
 (segment (start 101.6 85.0519) (end 101.5619 85.0138) (width 0.508) (layer F.Cu) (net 5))
 (segment (start 104.14 86.233) (end 104.14 86.4743) (width 0.25) (layer F.Cu) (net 6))
 (segment (start 104.14 88.9) (end 104.14 86.4743) (width 0.508) (layer F.Cu) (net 6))
 (segment (start 101.5746 83.1723) (end 102.3326 83.1723) (width 0.25) (layer F.Cu) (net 6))
 (segment (start 102.3326 83.1723) (end 102.9843 83.824) (width 0.25) (layer F.Cu) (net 6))
 (segment (start 102.9843 83.824) (end 102.9843 85.0773) (width 0.25) (layer F.Cu) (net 6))
 (segment (start 102.9843 85.0773) (end 104.14 86.233) (width 0.25) (layer F.Cu) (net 6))
 (segment (start 101.5746 82.4143) (end 101.5746 83.1723) (width 0.25) (layer F.Cu) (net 6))
 (segment (start 104.043798 81.824998) (end 102.163902 81.824998) (width 0.25) (layer F.Cu) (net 6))
 (segment (start 102.163902 81.824998) (end 101.5746 82.4143) (width 0.25) (layer F.Cu) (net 6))
 (segment (start 104.139 81.9202) (end 104.043798 81.824998) (width 0.25) (layer F.Cu) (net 6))
 (segment (start 104.639 81.9202) (end 104.139 81.9202) (width 0.25) (layer F.Cu) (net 6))
 (segment (start 105.41 80.2386) (end 105.41 81.6492) (width 0.25) (layer F.Cu) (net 6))
 (segment (start 105.41 75.818222) (end 105.41 78.231222) (width 0.508) (layer F.Cu) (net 6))
 (segment (start 105.41 78.231222) (end 105.41 80.2386) (width 0.508) (layer F.Cu) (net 6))
 (segment (start 105.41 81.6492) (end 105.139 81.9202) (width 0.25) (layer F.Cu) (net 6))
 (segment (start 105.139 81.9202) (end 104.639 81.9202) (width 0.25) (layer F.Cu) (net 6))
 (segment (start 106.689 81.2702) (end 106.9946 81.2702) (width 0.25) (layer F.Cu) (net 11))
 (segment (start 109.2708 78.994) (end 111.4973 78.994) (width 0.25) (layer F.Cu) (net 11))
 (segment (start 106.9946 81.2702) (end 109.2708 78.994) (width 0.25) (layer F.Cu) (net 11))
 (segment (start 111.4973 78.994) (end 112.2466 79.7433) (width 0.25) (layer F.Cu) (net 11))
 (segment (start 112.2466 79.7433) (end 113.0046 79.7433) (width 0.25) (layer F.Cu) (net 11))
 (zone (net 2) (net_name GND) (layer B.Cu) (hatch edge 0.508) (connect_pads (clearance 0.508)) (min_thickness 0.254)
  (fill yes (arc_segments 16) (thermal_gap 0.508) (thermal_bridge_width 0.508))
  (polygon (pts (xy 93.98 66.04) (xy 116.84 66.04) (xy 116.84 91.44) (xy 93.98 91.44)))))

